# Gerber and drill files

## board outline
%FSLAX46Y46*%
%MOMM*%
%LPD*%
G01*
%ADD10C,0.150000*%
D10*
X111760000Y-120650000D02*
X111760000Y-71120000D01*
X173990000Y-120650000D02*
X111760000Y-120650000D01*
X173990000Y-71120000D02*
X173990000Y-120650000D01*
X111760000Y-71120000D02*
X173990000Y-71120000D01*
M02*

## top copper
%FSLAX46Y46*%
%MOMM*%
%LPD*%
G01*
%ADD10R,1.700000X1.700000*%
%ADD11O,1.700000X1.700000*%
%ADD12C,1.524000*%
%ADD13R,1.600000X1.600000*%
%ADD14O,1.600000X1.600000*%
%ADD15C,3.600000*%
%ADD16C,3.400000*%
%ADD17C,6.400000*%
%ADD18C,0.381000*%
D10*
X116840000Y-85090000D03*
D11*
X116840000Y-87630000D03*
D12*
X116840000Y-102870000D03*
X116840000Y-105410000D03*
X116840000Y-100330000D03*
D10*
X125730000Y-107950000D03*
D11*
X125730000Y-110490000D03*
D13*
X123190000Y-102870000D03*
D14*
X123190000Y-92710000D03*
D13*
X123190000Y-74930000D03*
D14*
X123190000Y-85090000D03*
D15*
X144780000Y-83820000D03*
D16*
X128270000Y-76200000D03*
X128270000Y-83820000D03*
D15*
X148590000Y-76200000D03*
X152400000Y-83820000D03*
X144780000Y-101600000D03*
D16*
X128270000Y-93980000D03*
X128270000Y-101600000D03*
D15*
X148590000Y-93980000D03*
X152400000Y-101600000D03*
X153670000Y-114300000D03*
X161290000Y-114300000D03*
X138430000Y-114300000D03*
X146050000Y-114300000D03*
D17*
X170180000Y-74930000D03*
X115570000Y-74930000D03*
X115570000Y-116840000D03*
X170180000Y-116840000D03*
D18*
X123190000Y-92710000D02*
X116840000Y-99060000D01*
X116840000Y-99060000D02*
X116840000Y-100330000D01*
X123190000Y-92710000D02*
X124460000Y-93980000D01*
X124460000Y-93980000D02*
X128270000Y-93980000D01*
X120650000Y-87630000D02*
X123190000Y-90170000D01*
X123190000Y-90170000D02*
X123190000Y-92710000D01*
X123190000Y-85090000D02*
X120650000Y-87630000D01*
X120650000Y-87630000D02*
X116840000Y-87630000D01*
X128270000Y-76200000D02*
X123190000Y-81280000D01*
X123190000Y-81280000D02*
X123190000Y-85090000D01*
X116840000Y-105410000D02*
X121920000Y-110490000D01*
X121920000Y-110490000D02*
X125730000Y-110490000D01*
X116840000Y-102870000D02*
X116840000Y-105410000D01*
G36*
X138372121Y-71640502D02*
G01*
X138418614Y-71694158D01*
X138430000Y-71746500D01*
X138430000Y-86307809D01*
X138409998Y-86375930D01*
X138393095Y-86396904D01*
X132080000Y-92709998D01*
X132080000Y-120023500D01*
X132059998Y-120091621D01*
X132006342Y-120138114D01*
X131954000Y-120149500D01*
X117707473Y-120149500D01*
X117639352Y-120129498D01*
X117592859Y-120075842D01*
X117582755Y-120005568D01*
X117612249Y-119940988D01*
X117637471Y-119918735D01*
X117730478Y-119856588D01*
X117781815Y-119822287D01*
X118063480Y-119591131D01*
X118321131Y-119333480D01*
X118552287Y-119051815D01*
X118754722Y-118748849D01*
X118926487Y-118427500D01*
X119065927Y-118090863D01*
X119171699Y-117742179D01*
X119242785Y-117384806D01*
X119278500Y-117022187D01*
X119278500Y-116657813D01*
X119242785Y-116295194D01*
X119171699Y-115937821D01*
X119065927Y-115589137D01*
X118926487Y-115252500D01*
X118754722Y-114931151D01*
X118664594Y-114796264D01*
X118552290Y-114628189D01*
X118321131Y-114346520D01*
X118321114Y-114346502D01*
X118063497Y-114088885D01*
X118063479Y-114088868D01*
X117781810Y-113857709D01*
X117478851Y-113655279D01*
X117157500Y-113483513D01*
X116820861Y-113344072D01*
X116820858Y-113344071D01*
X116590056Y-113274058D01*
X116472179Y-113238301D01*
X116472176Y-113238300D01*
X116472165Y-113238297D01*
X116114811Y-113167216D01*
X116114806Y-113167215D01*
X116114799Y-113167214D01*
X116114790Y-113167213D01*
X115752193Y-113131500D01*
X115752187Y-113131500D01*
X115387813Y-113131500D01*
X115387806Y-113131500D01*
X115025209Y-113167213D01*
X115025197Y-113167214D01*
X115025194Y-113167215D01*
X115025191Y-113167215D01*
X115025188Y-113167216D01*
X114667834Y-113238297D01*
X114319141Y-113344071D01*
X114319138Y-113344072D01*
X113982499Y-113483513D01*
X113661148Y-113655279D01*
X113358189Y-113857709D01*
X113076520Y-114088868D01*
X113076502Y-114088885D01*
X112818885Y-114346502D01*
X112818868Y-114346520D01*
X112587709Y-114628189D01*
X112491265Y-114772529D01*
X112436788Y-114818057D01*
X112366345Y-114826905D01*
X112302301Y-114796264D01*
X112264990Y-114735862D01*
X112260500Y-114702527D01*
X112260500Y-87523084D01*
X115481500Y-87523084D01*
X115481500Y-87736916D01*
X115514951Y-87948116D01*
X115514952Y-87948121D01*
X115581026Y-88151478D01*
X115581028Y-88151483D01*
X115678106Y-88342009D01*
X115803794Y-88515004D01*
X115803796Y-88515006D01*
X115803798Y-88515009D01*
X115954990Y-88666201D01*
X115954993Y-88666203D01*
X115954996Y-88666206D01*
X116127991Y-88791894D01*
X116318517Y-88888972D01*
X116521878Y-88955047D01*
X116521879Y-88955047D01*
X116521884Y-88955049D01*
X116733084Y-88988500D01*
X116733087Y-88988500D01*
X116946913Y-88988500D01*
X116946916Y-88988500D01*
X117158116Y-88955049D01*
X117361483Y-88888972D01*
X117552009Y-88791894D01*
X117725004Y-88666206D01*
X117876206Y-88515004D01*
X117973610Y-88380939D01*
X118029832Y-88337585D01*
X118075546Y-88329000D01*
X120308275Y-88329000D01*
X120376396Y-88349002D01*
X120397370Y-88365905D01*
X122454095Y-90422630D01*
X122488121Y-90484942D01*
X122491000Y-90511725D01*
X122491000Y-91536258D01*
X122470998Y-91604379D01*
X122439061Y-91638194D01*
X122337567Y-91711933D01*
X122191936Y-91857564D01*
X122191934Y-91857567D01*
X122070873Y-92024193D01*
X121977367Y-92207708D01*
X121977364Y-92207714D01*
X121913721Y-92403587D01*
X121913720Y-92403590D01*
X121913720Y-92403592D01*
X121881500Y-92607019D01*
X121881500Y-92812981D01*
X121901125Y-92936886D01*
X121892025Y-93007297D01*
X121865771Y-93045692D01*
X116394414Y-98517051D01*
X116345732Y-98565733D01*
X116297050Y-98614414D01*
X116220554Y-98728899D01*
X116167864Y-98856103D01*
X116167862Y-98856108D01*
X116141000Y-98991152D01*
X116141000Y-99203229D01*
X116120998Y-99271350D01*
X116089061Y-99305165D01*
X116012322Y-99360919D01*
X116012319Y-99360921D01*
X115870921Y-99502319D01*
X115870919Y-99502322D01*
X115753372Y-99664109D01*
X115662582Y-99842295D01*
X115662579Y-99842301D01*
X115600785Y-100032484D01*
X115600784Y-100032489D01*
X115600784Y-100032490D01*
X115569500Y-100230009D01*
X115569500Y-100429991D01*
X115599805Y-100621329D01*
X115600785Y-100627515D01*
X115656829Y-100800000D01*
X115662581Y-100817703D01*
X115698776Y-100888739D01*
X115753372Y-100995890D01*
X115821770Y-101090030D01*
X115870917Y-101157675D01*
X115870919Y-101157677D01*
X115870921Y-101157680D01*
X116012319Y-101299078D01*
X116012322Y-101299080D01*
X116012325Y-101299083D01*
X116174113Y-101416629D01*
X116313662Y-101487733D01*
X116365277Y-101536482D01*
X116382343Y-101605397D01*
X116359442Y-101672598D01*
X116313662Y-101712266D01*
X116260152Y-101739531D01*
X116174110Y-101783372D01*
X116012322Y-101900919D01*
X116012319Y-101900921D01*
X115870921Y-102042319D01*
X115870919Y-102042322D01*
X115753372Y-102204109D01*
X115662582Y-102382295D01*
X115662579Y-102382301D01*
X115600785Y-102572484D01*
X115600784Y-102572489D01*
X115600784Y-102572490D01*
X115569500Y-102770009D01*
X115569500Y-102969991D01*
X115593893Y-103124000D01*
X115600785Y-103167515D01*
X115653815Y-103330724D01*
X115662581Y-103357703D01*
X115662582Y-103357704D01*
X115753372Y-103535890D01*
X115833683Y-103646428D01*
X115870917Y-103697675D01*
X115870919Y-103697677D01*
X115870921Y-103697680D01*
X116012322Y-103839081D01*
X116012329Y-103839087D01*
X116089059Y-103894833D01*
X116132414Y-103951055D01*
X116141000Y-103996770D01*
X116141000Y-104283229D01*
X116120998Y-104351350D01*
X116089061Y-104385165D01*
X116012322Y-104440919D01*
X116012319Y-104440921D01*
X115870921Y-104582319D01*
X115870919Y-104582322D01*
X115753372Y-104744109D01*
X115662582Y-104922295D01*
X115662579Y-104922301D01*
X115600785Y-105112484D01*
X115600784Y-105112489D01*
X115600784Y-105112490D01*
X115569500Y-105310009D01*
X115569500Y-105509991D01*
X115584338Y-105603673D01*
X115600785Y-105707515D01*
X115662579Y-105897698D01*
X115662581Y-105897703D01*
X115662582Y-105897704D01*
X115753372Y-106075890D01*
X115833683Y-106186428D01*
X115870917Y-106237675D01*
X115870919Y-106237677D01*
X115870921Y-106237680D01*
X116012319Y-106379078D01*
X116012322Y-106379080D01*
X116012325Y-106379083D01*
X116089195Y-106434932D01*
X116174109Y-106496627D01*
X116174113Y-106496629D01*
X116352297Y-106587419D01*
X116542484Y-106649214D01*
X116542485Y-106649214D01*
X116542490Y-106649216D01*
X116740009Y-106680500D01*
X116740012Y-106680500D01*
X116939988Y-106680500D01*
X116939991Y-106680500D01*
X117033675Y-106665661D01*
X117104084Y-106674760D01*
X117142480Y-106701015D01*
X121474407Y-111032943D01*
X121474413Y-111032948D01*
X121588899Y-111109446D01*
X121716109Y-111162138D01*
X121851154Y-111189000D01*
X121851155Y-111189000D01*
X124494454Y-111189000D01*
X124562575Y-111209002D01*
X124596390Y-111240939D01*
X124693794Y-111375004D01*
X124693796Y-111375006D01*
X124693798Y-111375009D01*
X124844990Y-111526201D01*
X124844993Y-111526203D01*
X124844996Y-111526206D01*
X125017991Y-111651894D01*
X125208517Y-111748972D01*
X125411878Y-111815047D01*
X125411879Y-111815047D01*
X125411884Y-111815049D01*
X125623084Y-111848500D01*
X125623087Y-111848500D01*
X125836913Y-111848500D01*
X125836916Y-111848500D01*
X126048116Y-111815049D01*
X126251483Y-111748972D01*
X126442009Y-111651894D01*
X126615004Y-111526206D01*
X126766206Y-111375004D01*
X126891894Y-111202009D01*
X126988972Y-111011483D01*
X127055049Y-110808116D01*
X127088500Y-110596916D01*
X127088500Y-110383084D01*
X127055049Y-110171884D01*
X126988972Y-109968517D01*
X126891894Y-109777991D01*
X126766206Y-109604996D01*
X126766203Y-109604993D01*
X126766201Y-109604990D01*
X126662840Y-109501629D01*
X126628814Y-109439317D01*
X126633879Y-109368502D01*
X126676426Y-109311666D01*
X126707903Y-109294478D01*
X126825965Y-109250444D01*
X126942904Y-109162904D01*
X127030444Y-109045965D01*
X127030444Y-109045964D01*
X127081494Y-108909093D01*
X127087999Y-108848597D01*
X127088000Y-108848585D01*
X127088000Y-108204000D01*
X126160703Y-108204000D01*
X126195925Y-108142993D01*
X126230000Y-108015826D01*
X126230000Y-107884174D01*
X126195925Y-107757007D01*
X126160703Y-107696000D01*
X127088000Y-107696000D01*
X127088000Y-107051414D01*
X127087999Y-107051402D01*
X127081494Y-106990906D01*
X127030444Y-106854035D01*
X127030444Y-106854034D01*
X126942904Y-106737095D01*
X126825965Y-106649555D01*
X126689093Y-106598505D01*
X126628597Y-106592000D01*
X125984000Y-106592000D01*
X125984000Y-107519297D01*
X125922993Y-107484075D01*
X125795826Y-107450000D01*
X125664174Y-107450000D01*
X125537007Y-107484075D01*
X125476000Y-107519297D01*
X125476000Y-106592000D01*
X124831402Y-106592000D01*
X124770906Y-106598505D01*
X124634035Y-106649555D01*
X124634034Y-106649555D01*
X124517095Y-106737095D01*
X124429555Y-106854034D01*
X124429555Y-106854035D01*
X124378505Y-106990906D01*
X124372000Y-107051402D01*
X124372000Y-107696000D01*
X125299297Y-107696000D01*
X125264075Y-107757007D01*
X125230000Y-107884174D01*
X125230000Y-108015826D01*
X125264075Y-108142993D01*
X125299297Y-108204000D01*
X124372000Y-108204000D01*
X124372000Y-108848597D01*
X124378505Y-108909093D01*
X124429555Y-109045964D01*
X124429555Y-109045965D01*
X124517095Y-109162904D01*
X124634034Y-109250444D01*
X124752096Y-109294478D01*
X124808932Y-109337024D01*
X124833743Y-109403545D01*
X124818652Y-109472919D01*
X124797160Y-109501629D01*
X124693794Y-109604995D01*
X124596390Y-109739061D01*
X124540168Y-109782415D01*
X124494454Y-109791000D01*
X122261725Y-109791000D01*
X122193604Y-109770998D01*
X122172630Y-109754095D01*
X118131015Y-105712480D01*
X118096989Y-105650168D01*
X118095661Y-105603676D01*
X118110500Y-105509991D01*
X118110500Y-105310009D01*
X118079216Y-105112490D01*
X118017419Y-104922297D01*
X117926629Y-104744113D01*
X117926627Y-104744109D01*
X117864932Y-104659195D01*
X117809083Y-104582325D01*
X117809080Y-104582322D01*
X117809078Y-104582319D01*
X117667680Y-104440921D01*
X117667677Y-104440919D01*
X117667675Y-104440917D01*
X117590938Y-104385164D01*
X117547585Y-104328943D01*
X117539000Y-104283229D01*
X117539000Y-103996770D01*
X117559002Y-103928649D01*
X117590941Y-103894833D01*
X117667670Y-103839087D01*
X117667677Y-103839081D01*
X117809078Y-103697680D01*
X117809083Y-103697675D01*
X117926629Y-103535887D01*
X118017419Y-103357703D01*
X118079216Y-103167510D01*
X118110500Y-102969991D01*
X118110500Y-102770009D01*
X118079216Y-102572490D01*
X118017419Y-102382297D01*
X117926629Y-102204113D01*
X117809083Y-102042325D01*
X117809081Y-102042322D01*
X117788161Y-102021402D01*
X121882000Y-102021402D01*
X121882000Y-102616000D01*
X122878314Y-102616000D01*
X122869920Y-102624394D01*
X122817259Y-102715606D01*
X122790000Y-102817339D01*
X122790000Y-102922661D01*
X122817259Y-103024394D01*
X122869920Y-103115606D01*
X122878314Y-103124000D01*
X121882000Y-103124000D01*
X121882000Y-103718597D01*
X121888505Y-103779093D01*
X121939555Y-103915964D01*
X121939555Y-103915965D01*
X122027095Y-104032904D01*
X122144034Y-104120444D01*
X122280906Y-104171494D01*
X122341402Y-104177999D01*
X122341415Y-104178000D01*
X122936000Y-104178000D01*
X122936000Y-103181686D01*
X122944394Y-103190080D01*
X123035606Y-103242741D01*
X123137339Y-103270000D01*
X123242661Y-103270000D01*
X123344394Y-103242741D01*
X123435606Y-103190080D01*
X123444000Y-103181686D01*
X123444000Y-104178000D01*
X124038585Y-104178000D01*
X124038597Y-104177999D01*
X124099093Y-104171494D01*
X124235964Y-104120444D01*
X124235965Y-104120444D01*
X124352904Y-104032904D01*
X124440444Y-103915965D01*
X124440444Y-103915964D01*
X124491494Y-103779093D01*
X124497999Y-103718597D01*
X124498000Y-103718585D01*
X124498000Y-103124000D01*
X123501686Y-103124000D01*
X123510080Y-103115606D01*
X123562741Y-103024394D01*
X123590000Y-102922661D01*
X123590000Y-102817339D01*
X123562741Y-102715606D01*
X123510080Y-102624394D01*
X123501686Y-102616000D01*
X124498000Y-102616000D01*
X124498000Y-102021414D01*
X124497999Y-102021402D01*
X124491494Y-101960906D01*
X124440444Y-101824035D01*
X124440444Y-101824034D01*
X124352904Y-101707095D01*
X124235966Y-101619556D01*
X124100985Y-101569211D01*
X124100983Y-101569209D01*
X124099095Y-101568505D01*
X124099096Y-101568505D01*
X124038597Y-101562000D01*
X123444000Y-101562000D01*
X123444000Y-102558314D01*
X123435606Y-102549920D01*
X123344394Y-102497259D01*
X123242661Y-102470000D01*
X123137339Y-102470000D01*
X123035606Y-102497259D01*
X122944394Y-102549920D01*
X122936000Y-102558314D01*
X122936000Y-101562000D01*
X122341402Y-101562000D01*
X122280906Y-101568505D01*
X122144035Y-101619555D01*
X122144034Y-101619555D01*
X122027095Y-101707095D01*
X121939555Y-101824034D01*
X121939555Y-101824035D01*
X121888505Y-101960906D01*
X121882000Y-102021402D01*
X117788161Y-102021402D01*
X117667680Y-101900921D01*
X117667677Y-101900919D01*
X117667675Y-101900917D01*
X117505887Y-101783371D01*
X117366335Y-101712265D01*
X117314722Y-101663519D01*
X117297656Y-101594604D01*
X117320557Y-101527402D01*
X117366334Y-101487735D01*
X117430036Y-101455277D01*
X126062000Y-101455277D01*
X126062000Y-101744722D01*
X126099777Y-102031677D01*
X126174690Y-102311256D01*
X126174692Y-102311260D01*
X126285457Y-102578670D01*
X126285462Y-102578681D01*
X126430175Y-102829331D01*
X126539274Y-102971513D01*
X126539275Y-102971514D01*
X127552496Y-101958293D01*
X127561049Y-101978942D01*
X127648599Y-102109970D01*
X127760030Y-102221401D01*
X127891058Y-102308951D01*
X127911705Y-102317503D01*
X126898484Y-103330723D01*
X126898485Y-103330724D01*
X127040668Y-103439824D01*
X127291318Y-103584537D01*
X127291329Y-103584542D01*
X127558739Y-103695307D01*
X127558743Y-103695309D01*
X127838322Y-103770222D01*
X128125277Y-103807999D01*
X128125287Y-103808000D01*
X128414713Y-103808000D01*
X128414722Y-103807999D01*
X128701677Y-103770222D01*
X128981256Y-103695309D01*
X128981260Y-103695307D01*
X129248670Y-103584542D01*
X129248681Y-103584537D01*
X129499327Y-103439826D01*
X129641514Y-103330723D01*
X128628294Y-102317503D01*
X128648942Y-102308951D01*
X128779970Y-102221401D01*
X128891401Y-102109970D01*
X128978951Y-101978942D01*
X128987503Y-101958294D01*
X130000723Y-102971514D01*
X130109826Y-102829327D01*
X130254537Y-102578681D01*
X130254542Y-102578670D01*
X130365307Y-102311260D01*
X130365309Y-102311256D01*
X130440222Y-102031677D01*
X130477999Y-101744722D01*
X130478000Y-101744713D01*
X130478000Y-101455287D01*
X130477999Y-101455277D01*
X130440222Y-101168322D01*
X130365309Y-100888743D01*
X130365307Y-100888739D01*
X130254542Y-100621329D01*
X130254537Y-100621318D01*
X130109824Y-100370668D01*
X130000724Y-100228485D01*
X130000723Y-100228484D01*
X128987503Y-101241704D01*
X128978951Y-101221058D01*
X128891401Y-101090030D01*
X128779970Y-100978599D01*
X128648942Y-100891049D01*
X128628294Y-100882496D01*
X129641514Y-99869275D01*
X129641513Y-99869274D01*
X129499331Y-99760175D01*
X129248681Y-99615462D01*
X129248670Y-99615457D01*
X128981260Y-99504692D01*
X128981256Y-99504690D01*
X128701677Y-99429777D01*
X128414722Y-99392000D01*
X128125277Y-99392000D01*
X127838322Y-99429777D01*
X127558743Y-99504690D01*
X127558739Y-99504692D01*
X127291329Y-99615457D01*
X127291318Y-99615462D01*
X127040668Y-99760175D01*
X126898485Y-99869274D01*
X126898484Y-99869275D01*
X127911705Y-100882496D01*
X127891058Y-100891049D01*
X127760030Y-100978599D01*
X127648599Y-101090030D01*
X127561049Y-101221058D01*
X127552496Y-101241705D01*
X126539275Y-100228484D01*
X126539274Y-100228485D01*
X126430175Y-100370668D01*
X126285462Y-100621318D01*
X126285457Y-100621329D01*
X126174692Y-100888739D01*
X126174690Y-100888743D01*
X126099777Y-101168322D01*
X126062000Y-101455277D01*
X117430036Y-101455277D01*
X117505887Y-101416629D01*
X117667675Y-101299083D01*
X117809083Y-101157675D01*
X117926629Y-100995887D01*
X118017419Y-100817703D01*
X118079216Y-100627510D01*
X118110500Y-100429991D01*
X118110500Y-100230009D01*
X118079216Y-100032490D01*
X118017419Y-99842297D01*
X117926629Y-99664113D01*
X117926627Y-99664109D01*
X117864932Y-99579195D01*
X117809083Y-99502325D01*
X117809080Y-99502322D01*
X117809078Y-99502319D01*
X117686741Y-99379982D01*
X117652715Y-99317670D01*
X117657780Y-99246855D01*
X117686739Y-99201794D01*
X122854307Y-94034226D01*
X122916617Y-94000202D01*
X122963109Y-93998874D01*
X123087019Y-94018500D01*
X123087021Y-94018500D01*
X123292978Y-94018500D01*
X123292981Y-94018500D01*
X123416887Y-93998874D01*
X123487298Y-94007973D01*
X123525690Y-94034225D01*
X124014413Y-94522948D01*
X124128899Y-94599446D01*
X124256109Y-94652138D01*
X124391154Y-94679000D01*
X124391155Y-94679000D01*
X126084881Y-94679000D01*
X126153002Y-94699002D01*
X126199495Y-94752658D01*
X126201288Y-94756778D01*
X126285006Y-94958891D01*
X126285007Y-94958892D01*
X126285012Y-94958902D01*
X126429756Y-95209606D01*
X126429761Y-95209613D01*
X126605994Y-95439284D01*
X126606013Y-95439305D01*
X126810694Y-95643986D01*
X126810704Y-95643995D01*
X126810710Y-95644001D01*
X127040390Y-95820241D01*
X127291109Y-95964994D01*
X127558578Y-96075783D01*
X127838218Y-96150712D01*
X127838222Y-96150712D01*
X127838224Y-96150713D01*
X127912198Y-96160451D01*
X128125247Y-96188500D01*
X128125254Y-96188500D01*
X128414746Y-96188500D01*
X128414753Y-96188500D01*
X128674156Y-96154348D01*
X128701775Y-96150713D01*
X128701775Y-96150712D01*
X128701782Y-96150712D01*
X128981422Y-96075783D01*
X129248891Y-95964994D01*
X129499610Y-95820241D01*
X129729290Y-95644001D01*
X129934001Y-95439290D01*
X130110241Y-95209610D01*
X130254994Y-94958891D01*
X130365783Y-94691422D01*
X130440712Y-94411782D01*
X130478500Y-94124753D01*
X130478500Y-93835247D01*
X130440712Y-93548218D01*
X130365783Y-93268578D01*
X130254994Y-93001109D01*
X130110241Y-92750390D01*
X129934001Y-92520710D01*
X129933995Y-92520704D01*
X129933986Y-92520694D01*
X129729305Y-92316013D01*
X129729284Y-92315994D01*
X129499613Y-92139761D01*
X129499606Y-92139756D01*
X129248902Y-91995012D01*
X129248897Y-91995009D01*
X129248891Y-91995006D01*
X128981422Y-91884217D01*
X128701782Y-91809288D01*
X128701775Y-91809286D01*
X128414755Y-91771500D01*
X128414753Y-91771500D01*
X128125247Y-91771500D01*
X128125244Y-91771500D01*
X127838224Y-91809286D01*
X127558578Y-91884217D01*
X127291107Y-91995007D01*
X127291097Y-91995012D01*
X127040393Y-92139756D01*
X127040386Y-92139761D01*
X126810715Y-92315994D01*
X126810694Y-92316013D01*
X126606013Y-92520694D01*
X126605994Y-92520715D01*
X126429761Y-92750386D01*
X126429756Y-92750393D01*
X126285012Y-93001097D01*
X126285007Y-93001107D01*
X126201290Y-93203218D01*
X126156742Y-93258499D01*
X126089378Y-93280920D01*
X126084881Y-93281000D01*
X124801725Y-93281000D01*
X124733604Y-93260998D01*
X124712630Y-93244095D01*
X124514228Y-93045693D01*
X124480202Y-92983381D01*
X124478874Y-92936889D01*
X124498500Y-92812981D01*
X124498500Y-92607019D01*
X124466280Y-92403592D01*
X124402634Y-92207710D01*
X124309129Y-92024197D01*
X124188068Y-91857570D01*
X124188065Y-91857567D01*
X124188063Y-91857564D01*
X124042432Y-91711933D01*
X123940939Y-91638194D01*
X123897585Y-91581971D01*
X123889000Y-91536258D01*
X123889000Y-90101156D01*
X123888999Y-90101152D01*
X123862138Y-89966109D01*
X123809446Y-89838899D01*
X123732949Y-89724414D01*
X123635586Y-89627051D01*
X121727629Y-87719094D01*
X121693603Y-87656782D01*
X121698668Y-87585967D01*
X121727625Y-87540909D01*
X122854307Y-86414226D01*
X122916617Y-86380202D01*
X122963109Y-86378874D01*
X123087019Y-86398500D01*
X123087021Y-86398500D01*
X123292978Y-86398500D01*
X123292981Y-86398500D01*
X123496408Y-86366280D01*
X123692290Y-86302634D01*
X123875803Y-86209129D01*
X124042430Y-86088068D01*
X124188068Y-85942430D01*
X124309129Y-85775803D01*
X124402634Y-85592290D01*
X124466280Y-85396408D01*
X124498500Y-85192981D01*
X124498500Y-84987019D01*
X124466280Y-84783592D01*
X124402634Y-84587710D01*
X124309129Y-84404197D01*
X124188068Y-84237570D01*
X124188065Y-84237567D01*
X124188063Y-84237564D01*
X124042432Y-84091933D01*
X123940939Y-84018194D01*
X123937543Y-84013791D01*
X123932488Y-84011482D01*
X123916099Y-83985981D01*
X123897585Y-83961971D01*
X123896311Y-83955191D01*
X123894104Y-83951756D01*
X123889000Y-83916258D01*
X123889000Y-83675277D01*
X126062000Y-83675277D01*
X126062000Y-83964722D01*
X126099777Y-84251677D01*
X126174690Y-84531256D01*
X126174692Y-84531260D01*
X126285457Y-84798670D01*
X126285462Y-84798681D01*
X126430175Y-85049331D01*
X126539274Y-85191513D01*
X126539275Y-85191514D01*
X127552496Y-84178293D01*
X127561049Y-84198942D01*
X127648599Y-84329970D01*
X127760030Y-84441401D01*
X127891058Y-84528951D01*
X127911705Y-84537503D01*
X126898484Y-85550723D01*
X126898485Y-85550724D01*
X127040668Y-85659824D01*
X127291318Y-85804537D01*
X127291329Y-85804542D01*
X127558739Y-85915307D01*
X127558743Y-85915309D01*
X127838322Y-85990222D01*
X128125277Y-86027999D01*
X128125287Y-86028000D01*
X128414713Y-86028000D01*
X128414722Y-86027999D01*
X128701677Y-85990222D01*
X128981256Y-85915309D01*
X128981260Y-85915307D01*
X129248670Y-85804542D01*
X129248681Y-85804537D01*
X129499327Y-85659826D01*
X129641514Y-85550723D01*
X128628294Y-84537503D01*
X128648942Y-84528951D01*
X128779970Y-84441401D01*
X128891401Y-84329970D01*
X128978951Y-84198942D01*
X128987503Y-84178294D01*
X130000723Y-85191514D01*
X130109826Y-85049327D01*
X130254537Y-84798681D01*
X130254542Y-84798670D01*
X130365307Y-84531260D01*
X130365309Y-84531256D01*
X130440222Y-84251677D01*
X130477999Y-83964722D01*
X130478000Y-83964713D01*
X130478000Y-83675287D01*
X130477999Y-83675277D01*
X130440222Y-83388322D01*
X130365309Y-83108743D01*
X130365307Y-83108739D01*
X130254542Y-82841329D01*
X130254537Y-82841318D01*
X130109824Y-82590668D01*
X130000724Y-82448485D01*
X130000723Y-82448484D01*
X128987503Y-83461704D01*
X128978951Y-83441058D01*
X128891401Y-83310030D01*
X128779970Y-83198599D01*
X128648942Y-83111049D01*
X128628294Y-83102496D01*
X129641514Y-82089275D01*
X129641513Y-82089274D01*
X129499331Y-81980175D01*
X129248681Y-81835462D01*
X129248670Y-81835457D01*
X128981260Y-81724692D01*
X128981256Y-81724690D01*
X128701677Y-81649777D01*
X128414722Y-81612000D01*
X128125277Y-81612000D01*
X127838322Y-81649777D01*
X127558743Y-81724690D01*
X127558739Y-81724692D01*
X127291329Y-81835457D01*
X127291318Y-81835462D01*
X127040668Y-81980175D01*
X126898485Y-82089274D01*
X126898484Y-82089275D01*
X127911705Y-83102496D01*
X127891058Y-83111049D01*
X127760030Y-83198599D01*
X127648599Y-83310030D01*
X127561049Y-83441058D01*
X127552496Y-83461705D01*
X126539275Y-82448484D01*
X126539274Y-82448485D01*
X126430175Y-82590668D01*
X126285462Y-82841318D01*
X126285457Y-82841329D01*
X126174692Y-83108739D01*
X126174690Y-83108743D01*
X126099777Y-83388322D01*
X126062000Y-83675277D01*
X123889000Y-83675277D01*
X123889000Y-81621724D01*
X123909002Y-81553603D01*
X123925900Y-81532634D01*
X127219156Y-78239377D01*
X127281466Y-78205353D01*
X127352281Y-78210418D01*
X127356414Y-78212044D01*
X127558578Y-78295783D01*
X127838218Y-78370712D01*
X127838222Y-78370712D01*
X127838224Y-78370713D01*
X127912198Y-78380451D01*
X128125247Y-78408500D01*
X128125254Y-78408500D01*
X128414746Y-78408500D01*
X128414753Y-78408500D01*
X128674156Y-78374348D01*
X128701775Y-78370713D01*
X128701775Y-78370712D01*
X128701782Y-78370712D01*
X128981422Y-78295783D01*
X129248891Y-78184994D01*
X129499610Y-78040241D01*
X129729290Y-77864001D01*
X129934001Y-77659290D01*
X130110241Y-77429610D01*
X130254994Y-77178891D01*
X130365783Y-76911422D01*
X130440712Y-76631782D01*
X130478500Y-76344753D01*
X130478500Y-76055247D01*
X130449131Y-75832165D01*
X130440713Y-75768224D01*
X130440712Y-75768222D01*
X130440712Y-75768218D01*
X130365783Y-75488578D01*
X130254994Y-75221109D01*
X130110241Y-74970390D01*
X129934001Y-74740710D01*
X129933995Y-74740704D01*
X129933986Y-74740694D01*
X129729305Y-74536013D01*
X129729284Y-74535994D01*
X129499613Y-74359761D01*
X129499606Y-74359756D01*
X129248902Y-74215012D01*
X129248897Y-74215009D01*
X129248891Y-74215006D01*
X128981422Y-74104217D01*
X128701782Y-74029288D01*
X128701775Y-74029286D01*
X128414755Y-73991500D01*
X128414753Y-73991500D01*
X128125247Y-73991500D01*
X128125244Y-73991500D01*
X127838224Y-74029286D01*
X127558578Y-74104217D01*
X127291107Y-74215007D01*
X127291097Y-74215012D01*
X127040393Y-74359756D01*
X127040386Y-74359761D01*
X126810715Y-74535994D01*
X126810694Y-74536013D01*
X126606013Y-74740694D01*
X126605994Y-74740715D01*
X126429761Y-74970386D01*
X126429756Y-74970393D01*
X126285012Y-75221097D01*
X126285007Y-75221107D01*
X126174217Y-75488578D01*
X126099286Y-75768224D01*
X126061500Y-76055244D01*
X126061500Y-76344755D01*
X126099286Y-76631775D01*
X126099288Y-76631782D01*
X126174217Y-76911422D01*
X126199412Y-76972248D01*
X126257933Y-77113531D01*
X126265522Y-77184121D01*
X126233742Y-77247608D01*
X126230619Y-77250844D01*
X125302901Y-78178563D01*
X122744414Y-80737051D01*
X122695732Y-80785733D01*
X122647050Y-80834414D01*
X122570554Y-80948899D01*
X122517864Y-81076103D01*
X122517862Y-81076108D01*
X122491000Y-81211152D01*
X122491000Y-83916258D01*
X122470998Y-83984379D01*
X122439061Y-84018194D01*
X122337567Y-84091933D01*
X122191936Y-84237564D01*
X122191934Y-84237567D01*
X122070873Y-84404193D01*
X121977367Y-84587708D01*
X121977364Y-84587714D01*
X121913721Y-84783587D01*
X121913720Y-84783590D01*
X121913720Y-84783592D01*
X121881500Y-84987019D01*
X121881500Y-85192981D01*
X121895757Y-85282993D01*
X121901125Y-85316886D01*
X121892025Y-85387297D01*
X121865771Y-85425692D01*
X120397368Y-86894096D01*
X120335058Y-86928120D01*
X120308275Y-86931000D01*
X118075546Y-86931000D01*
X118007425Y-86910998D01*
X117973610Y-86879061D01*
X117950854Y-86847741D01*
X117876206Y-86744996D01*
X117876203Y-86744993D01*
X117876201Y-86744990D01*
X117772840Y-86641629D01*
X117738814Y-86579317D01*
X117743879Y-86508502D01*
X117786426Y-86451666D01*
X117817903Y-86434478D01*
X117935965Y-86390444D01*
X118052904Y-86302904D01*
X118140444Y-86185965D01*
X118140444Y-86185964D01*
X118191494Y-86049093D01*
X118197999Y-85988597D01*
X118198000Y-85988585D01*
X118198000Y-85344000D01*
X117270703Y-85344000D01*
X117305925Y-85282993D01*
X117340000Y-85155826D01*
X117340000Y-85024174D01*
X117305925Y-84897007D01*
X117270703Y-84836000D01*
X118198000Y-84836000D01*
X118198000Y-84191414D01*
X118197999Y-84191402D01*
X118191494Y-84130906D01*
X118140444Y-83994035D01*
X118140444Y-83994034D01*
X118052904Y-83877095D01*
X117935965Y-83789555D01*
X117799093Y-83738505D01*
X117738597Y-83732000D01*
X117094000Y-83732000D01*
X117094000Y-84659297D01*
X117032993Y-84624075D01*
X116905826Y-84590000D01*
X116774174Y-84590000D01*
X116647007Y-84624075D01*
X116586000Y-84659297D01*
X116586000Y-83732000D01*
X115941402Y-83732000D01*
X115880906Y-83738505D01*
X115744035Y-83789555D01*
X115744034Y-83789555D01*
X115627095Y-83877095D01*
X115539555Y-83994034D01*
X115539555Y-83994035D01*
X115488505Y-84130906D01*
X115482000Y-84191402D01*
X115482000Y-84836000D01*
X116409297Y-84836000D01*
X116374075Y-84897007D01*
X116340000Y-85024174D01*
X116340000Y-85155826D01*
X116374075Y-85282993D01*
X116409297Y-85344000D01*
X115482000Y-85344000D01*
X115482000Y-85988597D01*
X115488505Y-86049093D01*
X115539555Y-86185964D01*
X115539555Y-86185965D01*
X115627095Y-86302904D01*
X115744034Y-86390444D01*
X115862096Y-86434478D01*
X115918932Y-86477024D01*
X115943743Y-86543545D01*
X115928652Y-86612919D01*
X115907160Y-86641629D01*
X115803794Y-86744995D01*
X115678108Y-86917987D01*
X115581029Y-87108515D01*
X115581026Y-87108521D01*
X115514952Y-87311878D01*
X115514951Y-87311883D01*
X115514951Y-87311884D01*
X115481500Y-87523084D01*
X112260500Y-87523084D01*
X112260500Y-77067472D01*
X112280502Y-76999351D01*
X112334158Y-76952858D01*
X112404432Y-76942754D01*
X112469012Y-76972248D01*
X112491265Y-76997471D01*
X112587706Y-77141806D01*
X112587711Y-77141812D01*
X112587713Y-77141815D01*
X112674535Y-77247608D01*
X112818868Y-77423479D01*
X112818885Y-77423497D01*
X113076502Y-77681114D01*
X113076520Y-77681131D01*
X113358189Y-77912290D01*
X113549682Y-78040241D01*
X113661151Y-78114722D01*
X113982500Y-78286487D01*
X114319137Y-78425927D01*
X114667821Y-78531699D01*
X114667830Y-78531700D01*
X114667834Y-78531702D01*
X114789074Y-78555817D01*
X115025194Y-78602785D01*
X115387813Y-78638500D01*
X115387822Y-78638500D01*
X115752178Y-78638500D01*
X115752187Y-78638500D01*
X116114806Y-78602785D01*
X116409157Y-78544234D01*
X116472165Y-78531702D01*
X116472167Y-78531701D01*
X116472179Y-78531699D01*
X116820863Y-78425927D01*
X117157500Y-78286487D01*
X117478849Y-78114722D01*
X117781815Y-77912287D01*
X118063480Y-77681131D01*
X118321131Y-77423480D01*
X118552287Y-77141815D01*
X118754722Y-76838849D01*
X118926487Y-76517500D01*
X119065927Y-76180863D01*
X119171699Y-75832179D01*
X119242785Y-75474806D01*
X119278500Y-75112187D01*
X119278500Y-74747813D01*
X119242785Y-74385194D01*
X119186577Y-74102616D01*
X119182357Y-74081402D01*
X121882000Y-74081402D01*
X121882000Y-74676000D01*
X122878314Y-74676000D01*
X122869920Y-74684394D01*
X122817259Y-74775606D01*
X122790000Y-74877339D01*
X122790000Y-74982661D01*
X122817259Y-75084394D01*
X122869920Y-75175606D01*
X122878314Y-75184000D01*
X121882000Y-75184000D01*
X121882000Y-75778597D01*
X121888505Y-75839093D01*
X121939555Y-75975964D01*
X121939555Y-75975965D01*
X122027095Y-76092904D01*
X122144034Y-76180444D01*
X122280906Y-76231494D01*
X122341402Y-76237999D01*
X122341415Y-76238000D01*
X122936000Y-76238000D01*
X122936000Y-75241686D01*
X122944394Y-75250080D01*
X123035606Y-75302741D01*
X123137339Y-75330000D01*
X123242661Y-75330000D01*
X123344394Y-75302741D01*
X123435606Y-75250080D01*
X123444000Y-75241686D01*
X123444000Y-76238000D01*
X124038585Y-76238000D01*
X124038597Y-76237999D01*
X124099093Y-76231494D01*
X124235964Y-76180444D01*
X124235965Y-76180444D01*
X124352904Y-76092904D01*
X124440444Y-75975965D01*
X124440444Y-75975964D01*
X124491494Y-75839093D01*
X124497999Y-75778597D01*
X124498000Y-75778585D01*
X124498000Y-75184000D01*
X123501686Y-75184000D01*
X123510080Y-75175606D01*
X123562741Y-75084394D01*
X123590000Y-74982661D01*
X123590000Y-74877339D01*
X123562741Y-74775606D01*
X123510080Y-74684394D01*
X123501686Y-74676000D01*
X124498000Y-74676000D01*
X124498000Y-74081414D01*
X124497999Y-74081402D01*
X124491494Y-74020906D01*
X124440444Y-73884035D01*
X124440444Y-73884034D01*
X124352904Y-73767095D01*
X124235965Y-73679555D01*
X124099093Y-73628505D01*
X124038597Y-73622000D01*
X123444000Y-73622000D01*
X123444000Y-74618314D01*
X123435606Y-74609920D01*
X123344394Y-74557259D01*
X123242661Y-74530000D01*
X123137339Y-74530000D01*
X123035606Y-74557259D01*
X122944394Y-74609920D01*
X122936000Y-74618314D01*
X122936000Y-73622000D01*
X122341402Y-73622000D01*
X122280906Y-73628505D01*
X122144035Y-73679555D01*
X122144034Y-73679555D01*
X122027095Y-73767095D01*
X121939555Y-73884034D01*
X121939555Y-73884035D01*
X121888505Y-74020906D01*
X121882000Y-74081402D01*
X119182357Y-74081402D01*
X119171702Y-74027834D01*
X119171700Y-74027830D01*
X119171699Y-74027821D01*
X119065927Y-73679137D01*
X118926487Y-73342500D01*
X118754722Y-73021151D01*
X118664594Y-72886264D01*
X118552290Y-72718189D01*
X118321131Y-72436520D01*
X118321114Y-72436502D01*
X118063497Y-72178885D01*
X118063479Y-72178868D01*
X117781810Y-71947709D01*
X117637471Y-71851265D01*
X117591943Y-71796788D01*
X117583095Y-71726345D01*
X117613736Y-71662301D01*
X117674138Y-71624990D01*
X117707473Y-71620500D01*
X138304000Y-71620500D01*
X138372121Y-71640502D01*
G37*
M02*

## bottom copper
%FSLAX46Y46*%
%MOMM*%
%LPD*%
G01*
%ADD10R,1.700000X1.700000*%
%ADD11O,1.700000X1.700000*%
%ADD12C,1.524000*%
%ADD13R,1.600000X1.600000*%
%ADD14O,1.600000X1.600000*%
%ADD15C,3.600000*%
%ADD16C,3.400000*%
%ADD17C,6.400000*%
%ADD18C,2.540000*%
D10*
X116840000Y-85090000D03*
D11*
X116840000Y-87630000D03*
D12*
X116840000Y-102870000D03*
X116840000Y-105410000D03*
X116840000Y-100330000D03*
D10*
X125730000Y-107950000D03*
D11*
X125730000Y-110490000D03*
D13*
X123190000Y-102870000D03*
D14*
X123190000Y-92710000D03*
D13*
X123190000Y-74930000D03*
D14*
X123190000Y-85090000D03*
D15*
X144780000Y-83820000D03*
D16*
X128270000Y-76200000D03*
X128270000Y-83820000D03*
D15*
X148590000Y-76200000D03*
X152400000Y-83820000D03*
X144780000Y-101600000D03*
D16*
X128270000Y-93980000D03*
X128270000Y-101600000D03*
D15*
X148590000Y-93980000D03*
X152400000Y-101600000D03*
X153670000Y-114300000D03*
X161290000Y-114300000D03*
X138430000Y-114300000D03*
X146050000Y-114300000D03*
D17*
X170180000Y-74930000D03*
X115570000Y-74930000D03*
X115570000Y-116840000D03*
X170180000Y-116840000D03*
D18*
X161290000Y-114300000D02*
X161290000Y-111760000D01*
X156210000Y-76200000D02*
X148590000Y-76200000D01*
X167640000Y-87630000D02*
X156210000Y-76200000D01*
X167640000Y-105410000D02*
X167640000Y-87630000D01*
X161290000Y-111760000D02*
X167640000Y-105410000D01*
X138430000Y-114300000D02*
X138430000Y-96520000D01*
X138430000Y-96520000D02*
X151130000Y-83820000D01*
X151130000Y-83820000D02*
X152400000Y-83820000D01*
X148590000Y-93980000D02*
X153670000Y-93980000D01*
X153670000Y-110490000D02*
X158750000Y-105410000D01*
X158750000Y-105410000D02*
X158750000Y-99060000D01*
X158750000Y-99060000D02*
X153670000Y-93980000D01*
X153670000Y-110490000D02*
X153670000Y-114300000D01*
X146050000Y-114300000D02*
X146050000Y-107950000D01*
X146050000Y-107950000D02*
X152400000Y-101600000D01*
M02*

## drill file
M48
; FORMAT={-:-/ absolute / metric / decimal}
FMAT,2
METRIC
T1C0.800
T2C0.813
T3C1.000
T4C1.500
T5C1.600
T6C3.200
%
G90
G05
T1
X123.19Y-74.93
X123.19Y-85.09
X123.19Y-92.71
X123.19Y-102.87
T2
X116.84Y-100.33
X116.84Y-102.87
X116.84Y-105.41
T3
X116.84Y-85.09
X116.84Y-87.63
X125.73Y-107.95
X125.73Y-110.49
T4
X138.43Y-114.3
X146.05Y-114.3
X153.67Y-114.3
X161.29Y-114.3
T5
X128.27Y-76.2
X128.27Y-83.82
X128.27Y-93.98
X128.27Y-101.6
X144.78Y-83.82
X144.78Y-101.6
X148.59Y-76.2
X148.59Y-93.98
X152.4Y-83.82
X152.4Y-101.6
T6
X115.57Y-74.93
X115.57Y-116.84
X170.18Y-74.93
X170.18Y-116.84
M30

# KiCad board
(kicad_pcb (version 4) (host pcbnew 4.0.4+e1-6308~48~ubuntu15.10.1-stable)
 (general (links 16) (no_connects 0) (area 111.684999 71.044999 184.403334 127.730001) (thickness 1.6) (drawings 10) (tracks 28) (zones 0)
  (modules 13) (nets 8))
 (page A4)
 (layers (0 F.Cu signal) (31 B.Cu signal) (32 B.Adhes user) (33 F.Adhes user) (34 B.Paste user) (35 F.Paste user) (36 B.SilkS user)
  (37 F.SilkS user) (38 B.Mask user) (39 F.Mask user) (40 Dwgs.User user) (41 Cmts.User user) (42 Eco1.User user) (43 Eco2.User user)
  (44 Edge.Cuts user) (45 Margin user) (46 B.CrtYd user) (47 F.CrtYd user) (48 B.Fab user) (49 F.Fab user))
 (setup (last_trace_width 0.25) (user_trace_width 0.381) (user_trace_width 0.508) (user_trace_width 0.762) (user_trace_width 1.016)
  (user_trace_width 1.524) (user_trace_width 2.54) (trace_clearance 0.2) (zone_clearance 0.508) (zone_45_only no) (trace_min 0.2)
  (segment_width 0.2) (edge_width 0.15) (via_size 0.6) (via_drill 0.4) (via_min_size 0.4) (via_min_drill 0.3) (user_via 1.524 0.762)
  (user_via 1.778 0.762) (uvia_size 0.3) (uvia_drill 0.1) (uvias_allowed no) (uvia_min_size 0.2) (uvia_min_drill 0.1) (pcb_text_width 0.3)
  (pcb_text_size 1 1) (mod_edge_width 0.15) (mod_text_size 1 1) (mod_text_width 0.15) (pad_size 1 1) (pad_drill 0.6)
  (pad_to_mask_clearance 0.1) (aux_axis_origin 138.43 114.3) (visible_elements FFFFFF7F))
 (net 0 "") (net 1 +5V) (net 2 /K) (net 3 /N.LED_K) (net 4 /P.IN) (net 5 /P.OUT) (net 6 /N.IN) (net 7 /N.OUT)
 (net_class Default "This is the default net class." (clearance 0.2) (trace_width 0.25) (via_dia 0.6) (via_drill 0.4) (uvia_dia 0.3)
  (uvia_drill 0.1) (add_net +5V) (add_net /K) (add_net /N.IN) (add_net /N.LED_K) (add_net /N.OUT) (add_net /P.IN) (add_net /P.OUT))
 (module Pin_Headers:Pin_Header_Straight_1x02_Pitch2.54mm (layer F.Cu) (at 116.84 85.09)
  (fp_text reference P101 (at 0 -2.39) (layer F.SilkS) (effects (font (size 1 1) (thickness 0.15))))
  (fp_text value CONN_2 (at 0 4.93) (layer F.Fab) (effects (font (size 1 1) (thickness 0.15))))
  (pad 1 thru_hole rect (at 0 0) (size 1.7 1.7) (drill 1) (layers *.Cu *.Mask) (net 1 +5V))
  (pad 2 thru_hole oval (at 0 2.54) (size 1.7 1.7) (drill 1) (layers *.Cu *.Mask) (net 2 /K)))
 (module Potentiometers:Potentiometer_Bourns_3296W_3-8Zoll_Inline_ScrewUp (layer F.Cu) (at 116.84 100.33 180)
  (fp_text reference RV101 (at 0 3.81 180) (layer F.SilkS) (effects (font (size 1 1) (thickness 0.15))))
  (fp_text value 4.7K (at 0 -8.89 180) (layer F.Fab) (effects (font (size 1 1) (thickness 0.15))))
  (pad 2 thru_hole circle (at 0 -2.54 180) (size 1.524 1.524) (drill 0.8128) (layers *.Cu *.Mask) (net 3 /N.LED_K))
  (pad 3 thru_hole circle (at 0 -5.08 180) (size 1.524 1.524) (drill 0.8128) (layers *.Cu *.Mask) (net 3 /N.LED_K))
  (pad 1 thru_hole circle (at 0 0 180) (size 1.524 1.524) (drill 0.8128) (layers *.Cu *.Mask) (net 2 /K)))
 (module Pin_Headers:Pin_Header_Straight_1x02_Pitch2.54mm (layer F.Cu) (at 125.73 107.95)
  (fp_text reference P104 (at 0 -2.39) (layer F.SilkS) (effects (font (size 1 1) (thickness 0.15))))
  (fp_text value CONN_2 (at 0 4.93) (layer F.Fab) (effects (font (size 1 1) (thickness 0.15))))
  (pad 1 thru_hole rect (at 0 0) (size 1.7 1.7) (drill 1) (layers *.Cu *.Mask) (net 1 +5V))
  (pad 2 thru_hole oval (at 0 2.54) (size 1.7 1.7) (drill 1) (layers *.Cu *.Mask) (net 3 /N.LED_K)))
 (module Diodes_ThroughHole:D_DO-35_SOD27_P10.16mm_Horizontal (layer F.Cu) (at 123.19 102.87 90)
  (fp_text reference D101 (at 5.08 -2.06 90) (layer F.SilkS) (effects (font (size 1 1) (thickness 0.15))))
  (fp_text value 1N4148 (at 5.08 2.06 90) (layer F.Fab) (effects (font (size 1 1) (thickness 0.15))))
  (pad 1 thru_hole rect (at 0 0 90) (size 1.6 1.6) (drill 0.8) (layers *.Cu *.Mask) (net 1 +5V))
  (pad 2 thru_hole oval (at 10.16 0 90) (size 1.6 1.6) (drill 0.8) (layers *.Cu *.Mask) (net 2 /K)))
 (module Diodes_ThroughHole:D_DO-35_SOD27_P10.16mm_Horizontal (layer F.Cu) (at 123.19 74.93 270)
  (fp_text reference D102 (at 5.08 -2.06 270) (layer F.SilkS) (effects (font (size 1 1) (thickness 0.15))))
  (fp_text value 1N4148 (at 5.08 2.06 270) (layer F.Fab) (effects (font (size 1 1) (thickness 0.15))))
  (pad 1 thru_hole rect (at 0 0 270) (size 1.6 1.6) (drill 0.8) (layers *.Cu *.Mask) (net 1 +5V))
  (pad 2 thru_hole oval (at 10.16 0 270) (size 1.6 1.6) (drill 0.8) (layers *.Cu *.Mask) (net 2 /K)))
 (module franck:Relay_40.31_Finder (layer F.Cu) (at 128.27 83.82)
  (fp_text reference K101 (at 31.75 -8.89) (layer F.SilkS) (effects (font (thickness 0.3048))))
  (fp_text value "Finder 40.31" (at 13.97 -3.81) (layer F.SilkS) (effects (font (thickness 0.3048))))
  (pad 12 thru_hole circle (at 16.51 0) (size 3.6 3.6) (drill 1.6) (layers *.Cu *.Mask F.SilkS))
  (pad A2 thru_hole circle (at 0 -7.62) (size 3.4 3.4) (drill 1.6) (layers *.Cu *.Mask F.SilkS) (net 2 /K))
  (pad A1 thru_hole circle (at 0 0) (size 3.4 3.4) (drill 1.6) (layers *.Cu *.Mask F.SilkS) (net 1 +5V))
  (pad 11 thru_hole circle (at 20.32 -7.62) (size 3.6 3.6) (drill 1.6) (layers *.Cu *.Mask F.SilkS) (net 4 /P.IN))
  (pad 14 thru_hole circle (at 24.13 0) (size 3.6 3.6) (drill 1.6) (layers *.Cu *.Mask F.SilkS) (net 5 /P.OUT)))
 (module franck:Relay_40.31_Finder (layer F.Cu) (at 128.27 101.6)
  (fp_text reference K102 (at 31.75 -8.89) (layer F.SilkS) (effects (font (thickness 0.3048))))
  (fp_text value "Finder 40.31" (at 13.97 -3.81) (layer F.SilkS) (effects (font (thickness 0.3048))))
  (pad 12 thru_hole circle (at 16.51 0) (size 3.6 3.6) (drill 1.6) (layers *.Cu *.Mask F.SilkS))
  (pad A2 thru_hole circle (at 0 -7.62) (size 3.4 3.4) (drill 1.6) (layers *.Cu *.Mask F.SilkS) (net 2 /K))
  (pad A1 thru_hole circle (at 0 0) (size 3.4 3.4) (drill 1.6) (layers *.Cu *.Mask F.SilkS) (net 1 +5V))
  (pad 11 thru_hole circle (at 20.32 -7.62) (size 3.6 3.6) (drill 1.6) (layers *.Cu *.Mask F.SilkS) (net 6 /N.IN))
  (pad 14 thru_hole circle (at 24.13 0) (size 3.6 3.6) (drill 1.6) (layers *.Cu *.Mask F.SilkS) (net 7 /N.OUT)))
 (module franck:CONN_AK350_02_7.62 (layer F.Cu) (at 153.67 114.3)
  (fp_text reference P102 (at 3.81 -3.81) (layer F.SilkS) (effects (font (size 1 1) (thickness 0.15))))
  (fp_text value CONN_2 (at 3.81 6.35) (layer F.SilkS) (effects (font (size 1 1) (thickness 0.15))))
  (pad 1 thru_hole circle (at 0 0) (size 3.6 3.6) (drill 1.5) (layers *.Cu *.Mask) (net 6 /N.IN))
  (pad 2 thru_hole circle (at 7.62 0) (size 3.6 3.6) (drill 1.5) (layers *.Cu *.Mask) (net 4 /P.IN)))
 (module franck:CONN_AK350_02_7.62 (layer F.Cu) (at 138.43 114.3)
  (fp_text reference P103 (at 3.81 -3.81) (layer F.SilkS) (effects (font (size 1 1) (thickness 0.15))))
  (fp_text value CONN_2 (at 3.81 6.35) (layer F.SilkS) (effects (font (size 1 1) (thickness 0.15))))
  (pad 1 thru_hole circle (at 0 0) (size 3.6 3.6) (drill 1.5) (layers *.Cu *.Mask) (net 5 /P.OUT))
  (pad 2 thru_hole circle (at 7.62 0) (size 3.6 3.6) (drill 1.5) (layers *.Cu *.Mask) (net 7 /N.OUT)))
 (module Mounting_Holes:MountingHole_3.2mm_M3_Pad (layer F.Cu) (at 170.18 74.93)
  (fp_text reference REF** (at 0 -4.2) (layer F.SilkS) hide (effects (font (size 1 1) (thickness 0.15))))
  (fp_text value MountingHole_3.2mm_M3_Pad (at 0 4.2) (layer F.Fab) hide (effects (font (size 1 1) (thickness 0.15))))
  (pad 1 thru_hole circle (at 0 0) (size 6.4 6.4) (drill 3.2) (layers *.Cu *.Mask)))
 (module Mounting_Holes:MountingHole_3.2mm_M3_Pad (layer F.Cu) (at 115.57 74.93)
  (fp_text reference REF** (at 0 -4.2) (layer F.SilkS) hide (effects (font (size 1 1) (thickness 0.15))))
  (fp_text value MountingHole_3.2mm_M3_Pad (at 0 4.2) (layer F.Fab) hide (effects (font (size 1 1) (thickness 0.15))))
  (pad 1 thru_hole circle (at 0 0) (size 6.4 6.4) (drill 3.2) (layers *.Cu *.Mask)))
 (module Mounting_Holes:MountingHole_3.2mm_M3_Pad (layer F.Cu) (at 115.57 116.84)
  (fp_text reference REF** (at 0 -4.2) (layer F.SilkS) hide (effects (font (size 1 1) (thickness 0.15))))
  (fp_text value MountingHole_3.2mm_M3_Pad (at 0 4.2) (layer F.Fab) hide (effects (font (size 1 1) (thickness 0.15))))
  (pad 1 thru_hole circle (at 0 0) (size 6.4 6.4) (drill 3.2) (layers *.Cu *.Mask)))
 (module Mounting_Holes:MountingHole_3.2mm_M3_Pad (layer F.Cu) (at 170.18 116.84)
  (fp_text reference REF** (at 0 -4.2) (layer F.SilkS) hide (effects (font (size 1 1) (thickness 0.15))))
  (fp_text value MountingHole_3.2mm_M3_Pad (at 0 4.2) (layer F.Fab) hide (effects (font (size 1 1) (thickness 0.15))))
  (pad 1 thru_hole circle (at 0 0) (size 6.4 6.4) (drill 3.2) (layers *.Cu *.Mask)))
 (gr_line (start 111.76 120.65) (end 111.76 71.12) (angle 90) (layer Edge.Cuts) (width 0.15))
 (gr_line (start 173.99 120.65) (end 111.76 120.65) (angle 90) (layer Edge.Cuts) (width 0.15))
 (gr_line (start 173.99 71.12) (end 173.99 120.65) (angle 90) (layer Edge.Cuts) (width 0.15))
 (gr_line (start 111.76 71.12) (end 173.99 71.12) (angle 90) (layer Edge.Cuts) (width 0.15))
 (segment (start 123.19 92.71) (end 116.84 99.06) (width 0.381) (layer F.Cu) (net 2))
 (segment (start 116.84 99.06) (end 116.84 100.33) (width 0.381) (layer F.Cu) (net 2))
 (segment (start 123.19 92.71) (end 124.46 93.98) (width 0.381) (layer F.Cu) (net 2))
 (segment (start 124.46 93.98) (end 128.27 93.98) (width 0.381) (layer F.Cu) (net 2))
 (segment (start 120.65 87.63) (end 123.19 90.17) (width 0.381) (layer F.Cu) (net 2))
 (segment (start 123.19 90.17) (end 123.19 92.71) (width 0.381) (layer F.Cu) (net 2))
 (segment (start 123.19 85.09) (end 120.65 87.63) (width 0.381) (layer F.Cu) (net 2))
 (segment (start 120.65 87.63) (end 116.84 87.63) (width 0.381) (layer F.Cu) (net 2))
 (segment (start 128.27 76.2) (end 123.19 81.28) (width 0.381) (layer F.Cu) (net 2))
 (segment (start 123.19 81.28) (end 123.19 85.09) (width 0.381) (layer F.Cu) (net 2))
 (segment (start 161.29 114.3) (end 161.29 111.76) (width 2.54) (layer B.Cu) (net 4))
 (segment (start 156.21 76.2) (end 148.59 76.2) (width 2.54) (layer B.Cu) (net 4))
 (segment (start 167.64 87.63) (end 156.21 76.2) (width 2.54) (layer B.Cu) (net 4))
 (segment (start 167.64 105.41) (end 167.64 87.63) (width 2.54) (layer B.Cu) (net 4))
 (segment (start 161.29 111.76) (end 167.64 105.41) (width 2.54) (layer B.Cu) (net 4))
 (segment (start 138.43 114.3) (end 138.43 96.52) (width 2.54) (layer B.Cu) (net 5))
 (segment (start 138.43 96.52) (end 151.13 83.82) (width 2.54) (layer B.Cu) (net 5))
 (segment (start 151.13 83.82) (end 152.4 83.82) (width 2.54) (layer B.Cu) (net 5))
 (segment (start 148.59 93.98) (end 153.67 93.98) (width 2.54) (layer B.Cu) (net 6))
 (segment (start 153.67 110.49) (end 158.75 105.41) (width 2.54) (layer B.Cu) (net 6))
 (segment (start 158.75 105.41) (end 158.75 99.06) (width 2.54) (layer B.Cu) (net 6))
 (segment (start 158.75 99.06) (end 153.67 93.98) (width 2.54) (layer B.Cu) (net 6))
 (segment (start 153.67 110.49) (end 153.67 114.3) (width 2.54) (layer B.Cu) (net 6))
 (segment (start 146.05 114.3) (end 146.05 107.95) (width 2.54) (layer B.Cu) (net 7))
 (segment (start 146.05 107.95) (end 152.4 101.6) (width 2.54) (layer B.Cu) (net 7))
 (segment (start 116.84 105.41) (end 121.92 110.49) (width 0.381) (layer F.Cu) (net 3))
 (segment (start 121.92 110.49) (end 125.73 110.49) (width 0.381) (layer F.Cu) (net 3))
 (segment (start 116.84 102.87) (end 116.84 105.41) (width 0.381) (layer F.Cu) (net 3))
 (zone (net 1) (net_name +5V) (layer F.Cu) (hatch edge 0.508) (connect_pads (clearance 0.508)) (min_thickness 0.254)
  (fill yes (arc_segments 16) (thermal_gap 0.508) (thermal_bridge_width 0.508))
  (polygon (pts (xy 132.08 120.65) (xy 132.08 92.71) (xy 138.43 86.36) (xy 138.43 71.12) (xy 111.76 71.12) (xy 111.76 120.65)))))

